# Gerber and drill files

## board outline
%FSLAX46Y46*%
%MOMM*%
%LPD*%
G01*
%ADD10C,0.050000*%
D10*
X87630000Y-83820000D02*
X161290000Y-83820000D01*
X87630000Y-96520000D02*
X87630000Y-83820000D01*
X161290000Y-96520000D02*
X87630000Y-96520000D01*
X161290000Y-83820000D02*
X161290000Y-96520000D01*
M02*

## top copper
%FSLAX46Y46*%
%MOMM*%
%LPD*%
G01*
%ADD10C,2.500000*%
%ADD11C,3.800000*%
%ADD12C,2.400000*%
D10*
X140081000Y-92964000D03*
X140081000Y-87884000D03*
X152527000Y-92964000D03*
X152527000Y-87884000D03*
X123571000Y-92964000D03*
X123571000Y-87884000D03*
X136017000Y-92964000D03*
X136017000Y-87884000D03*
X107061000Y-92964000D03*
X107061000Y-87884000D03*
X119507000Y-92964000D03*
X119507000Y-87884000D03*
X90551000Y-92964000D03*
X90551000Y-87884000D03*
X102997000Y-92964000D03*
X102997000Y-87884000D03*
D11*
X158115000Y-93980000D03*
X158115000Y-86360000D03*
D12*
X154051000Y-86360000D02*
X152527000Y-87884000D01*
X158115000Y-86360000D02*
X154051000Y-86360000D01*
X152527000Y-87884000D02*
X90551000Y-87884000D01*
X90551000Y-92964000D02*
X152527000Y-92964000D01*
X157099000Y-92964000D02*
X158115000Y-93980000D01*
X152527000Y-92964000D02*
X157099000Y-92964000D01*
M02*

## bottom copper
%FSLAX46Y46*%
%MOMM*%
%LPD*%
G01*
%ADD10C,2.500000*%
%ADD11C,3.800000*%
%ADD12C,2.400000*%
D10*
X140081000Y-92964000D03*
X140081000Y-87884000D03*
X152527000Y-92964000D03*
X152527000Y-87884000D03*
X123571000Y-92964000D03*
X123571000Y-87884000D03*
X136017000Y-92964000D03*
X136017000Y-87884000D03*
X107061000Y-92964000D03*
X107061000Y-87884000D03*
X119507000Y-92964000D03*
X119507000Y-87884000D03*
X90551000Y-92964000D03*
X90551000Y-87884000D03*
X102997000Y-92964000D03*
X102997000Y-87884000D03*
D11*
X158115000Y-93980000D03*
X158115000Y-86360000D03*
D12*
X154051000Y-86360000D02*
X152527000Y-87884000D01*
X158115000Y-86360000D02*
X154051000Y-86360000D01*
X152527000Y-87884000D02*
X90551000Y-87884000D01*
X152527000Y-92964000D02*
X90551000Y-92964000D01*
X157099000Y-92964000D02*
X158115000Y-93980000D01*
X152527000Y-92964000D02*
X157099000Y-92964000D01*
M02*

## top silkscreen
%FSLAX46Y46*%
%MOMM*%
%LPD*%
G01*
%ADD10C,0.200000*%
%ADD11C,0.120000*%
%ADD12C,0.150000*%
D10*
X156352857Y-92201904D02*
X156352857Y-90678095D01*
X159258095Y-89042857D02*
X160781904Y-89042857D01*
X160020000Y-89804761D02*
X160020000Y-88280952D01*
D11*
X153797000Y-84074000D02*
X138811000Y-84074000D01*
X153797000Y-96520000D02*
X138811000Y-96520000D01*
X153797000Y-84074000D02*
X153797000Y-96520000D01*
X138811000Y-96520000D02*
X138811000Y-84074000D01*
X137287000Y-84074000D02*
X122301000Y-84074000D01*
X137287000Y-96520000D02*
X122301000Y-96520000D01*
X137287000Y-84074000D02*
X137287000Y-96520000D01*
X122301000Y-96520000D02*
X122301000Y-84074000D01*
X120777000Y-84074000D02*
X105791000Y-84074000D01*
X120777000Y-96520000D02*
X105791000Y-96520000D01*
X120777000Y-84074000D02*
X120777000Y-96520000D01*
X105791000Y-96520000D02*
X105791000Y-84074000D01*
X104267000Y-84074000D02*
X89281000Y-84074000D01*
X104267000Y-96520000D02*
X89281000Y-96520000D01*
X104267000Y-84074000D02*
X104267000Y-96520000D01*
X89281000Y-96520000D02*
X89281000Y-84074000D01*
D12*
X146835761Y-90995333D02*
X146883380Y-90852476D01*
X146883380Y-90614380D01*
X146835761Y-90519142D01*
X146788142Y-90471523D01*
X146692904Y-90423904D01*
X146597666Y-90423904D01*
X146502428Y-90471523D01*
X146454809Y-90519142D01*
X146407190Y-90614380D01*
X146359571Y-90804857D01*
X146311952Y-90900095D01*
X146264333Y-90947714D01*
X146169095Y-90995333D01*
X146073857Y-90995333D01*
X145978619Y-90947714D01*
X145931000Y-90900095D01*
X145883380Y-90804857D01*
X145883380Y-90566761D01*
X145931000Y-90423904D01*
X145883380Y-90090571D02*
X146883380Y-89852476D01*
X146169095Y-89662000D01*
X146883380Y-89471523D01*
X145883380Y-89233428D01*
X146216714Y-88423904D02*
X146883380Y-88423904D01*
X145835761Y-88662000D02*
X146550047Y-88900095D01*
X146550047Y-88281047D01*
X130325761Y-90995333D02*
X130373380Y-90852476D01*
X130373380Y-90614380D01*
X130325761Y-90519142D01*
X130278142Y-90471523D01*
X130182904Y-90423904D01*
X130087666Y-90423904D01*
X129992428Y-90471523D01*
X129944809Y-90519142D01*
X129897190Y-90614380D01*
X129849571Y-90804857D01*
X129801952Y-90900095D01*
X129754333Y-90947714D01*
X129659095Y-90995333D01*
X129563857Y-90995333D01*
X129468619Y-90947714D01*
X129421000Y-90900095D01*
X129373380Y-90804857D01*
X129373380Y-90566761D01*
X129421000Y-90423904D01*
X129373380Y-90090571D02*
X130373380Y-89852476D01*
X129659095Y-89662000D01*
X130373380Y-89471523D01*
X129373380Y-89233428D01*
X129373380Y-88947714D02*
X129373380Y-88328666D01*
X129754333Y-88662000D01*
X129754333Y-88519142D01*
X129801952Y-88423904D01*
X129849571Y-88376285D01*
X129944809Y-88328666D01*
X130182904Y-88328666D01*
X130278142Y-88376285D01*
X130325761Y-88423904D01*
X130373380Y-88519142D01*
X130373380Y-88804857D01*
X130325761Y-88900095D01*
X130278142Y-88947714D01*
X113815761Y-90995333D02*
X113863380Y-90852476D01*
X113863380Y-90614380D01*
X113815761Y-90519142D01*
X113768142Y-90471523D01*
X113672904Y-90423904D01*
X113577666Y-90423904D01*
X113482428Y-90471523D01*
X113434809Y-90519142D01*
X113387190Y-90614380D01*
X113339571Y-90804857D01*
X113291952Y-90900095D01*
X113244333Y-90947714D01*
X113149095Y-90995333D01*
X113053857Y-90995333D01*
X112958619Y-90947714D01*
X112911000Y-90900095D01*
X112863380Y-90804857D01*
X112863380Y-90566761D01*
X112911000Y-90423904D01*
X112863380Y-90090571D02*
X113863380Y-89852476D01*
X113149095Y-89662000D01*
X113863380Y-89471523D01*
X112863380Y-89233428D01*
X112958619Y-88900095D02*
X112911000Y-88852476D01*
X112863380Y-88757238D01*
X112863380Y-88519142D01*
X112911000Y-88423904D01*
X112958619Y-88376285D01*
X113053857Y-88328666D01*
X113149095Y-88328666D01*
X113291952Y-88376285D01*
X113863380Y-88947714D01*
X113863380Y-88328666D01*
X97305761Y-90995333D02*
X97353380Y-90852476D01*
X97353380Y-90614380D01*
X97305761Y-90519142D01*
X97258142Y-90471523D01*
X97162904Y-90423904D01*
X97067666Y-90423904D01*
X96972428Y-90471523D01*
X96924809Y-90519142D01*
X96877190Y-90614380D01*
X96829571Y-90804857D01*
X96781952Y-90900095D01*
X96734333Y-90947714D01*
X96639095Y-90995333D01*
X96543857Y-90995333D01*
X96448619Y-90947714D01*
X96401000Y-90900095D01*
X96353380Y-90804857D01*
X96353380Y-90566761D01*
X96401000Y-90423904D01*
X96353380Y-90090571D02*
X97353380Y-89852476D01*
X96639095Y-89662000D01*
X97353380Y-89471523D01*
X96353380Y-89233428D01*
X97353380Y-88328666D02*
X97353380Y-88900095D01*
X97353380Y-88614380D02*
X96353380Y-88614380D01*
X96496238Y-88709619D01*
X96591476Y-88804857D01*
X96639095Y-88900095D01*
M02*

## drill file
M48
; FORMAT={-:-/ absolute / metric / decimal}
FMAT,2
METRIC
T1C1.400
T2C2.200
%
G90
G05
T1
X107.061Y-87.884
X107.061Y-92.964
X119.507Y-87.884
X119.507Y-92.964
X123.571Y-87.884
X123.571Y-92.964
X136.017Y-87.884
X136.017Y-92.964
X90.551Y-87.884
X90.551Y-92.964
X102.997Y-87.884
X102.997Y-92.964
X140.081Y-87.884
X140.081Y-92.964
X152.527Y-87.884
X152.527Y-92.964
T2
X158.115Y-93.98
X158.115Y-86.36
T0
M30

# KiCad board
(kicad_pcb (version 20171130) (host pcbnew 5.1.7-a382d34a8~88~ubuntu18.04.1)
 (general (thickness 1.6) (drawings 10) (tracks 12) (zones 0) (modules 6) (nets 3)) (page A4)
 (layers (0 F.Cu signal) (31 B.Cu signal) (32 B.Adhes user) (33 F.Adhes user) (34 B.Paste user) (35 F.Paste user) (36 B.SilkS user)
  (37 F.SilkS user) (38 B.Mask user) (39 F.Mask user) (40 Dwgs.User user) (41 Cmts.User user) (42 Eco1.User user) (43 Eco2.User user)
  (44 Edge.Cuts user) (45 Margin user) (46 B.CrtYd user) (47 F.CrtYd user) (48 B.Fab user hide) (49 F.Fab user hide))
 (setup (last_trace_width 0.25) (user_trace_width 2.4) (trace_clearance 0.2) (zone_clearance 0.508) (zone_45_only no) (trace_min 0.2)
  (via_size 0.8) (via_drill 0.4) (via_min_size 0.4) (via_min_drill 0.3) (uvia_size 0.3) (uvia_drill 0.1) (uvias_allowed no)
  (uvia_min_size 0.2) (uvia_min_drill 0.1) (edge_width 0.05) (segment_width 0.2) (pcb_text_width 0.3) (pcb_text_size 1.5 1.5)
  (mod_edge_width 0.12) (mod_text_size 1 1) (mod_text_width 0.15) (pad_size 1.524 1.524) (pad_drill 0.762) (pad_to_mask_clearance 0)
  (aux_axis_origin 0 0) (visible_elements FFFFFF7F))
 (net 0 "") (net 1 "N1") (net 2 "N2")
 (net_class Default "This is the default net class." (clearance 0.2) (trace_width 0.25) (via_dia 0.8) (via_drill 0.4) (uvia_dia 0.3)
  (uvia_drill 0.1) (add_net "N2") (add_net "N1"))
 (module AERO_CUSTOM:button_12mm (layer F.Cu) (at 142.875 81.28)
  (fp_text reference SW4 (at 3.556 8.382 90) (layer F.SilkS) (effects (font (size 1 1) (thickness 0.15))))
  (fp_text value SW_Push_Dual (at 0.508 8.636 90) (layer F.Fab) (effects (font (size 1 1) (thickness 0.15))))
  (fp_line (start -4.064 15.24) (end -4.064 2.794) (layer F.SilkS) (width 0.12))
  (fp_line (start 10.922 2.794) (end 10.922 15.24) (layer F.SilkS) (width 0.12))
  (fp_line (start 10.922 15.24) (end -4.064 15.24) (layer F.SilkS) (width 0.12))
  (fp_line (start 10.922 2.794) (end -4.064 2.794) (layer F.SilkS) (width 0.12))
  (pad 4 thru_hole circle (at -2.794 11.684) (size 2.5 2.5) (drill 1.4) (layers *.Cu *.Mask) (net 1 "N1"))
  (pad 3 thru_hole circle (at -2.794 6.604) (size 2.5 2.5) (drill 1.4) (layers *.Cu *.Mask) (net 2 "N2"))
  (pad 2 thru_hole circle (at 9.652 11.684) (size 2.5 2.5) (drill 1.4) (layers *.Cu *.Mask) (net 1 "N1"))
  (pad 1 thru_hole circle (at 9.652 6.604) (size 2.5 2.5) (drill 1.4) (layers *.Cu *.Mask) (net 2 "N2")))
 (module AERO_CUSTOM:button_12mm (layer F.Cu) (at 126.365 81.28)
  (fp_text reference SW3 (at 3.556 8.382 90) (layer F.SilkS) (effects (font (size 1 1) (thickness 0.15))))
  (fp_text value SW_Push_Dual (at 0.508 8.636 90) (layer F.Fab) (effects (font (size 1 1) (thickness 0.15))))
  (fp_line (start -4.064 15.24) (end -4.064 2.794) (layer F.SilkS) (width 0.12))
  (fp_line (start 10.922 2.794) (end 10.922 15.24) (layer F.SilkS) (width 0.12))
  (fp_line (start 10.922 15.24) (end -4.064 15.24) (layer F.SilkS) (width 0.12))
  (fp_line (start 10.922 2.794) (end -4.064 2.794) (layer F.SilkS) (width 0.12))
  (pad 4 thru_hole circle (at -2.794 11.684) (size 2.5 2.5) (drill 1.4) (layers *.Cu *.Mask) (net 1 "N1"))
  (pad 3 thru_hole circle (at -2.794 6.604) (size 2.5 2.5) (drill 1.4) (layers *.Cu *.Mask) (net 2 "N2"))
  (pad 2 thru_hole circle (at 9.652 11.684) (size 2.5 2.5) (drill 1.4) (layers *.Cu *.Mask) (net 1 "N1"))
  (pad 1 thru_hole circle (at 9.652 6.604) (size 2.5 2.5) (drill 1.4) (layers *.Cu *.Mask) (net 2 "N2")))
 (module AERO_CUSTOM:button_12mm (layer F.Cu) (at 109.855 81.28)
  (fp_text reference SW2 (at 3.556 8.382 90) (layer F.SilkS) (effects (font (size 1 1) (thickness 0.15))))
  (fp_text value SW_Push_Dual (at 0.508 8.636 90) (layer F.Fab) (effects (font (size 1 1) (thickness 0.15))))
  (fp_line (start -4.064 15.24) (end -4.064 2.794) (layer F.SilkS) (width 0.12))
  (fp_line (start 10.922 2.794) (end 10.922 15.24) (layer F.SilkS) (width 0.12))
  (fp_line (start 10.922 15.24) (end -4.064 15.24) (layer F.SilkS) (width 0.12))
  (fp_line (start 10.922 2.794) (end -4.064 2.794) (layer F.SilkS) (width 0.12))
  (pad 4 thru_hole circle (at -2.794 11.684) (size 2.5 2.5) (drill 1.4) (layers *.Cu *.Mask) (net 1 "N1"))
  (pad 3 thru_hole circle (at -2.794 6.604) (size 2.5 2.5) (drill 1.4) (layers *.Cu *.Mask) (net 2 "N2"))
  (pad 2 thru_hole circle (at 9.652 11.684) (size 2.5 2.5) (drill 1.4) (layers *.Cu *.Mask) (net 1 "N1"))
  (pad 1 thru_hole circle (at 9.652 6.604) (size 2.5 2.5) (drill 1.4) (layers *.Cu *.Mask) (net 2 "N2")))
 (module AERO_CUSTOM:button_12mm (layer F.Cu) (at 93.345 81.28)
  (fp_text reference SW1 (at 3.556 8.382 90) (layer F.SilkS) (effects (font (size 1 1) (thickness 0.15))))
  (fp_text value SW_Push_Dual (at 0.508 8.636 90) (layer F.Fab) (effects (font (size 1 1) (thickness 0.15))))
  (fp_line (start -4.064 15.24) (end -4.064 2.794) (layer F.SilkS) (width 0.12))
  (fp_line (start 10.922 2.794) (end 10.922 15.24) (layer F.SilkS) (width 0.12))
  (fp_line (start 10.922 15.24) (end -4.064 15.24) (layer F.SilkS) (width 0.12))
  (fp_line (start 10.922 2.794) (end -4.064 2.794) (layer F.SilkS) (width 0.12))
  (pad 4 thru_hole circle (at -2.794 11.684) (size 2.5 2.5) (drill 1.4) (layers *.Cu *.Mask) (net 1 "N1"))
  (pad 3 thru_hole circle (at -2.794 6.604) (size 2.5 2.5) (drill 1.4) (layers *.Cu *.Mask) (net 2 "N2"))
  (pad 2 thru_hole circle (at 9.652 11.684) (size 2.5 2.5) (drill 1.4) (layers *.Cu *.Mask) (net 1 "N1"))
  (pad 1 thru_hole circle (at 9.652 6.604) (size 2.5 2.5) (drill 1.4) (layers *.Cu *.Mask) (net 2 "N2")))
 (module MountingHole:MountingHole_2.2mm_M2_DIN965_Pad (layer F.Cu) (at 158.115 93.98)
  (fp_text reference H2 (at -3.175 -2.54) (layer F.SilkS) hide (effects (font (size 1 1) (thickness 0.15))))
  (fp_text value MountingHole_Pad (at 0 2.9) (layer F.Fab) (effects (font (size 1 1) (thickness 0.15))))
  (pad 1 thru_hole circle (at 0 0) (size 3.8 3.8) (drill 2.2) (layers *.Cu *.Mask) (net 1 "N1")))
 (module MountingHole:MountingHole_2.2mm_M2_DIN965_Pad (layer F.Cu) (at 158.115 86.36)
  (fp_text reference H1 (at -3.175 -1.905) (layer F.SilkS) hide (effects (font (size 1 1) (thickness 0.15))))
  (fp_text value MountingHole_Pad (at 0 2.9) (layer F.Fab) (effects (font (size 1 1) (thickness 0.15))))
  (pad 1 thru_hole circle (at 0 0) (size 3.8 3.8) (drill 2.2) (layers *.Cu *.Mask) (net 2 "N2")))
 (gr_line (start 87.63 83.82) (end 161.29 83.82) (layer Edge.Cuts) (width 0.05))
 (gr_line (start 87.63 96.52) (end 87.63 83.82) (layer Edge.Cuts) (width 0.05))
 (gr_line (start 161.29 96.52) (end 87.63 96.52) (layer Edge.Cuts) (width 0.05))
 (gr_line (start 161.29 83.82) (end 161.29 96.52) (layer Edge.Cuts) (width 0.05))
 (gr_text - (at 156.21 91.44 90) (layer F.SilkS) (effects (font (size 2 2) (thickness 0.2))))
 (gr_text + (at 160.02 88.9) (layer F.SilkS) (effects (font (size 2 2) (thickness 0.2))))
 (segment (start 154.051 86.36) (end 152.527 87.884) (width 2.4) (layer F.Cu) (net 2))
 (segment (start 158.115 86.36) (end 154.051 86.36) (width 2.4) (layer F.Cu) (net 2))
 (segment (start 152.527 87.884) (end 90.551 87.884) (width 2.4) (layer F.Cu) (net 2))
 (segment (start 154.051 86.36) (end 152.527 87.884) (width 2.4) (layer B.Cu) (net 2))
 (segment (start 158.115 86.36) (end 154.051 86.36) (width 2.4) (layer B.Cu) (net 2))
 (segment (start 152.527 87.884) (end 90.551 87.884) (width 2.4) (layer B.Cu) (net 2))
 (segment (start 90.551 92.964) (end 152.527 92.964) (width 2.4) (layer F.Cu) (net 1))
 (segment (start 157.099 92.964) (end 158.115 93.98) (width 2.4) (layer F.Cu) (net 1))
 (segment (start 152.527 92.964) (end 157.099 92.964) (width 2.4) (layer F.Cu) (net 1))
 (segment (start 152.527 92.964) (end 90.551 92.964) (width 2.4) (layer B.Cu) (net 1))
 (segment (start 157.099 92.964) (end 158.115 93.98) (width 2.4) (layer B.Cu) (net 1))
 (segment (start 152.527 92.964) (end 157.099 92.964) (width 2.4) (layer B.Cu) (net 1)))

